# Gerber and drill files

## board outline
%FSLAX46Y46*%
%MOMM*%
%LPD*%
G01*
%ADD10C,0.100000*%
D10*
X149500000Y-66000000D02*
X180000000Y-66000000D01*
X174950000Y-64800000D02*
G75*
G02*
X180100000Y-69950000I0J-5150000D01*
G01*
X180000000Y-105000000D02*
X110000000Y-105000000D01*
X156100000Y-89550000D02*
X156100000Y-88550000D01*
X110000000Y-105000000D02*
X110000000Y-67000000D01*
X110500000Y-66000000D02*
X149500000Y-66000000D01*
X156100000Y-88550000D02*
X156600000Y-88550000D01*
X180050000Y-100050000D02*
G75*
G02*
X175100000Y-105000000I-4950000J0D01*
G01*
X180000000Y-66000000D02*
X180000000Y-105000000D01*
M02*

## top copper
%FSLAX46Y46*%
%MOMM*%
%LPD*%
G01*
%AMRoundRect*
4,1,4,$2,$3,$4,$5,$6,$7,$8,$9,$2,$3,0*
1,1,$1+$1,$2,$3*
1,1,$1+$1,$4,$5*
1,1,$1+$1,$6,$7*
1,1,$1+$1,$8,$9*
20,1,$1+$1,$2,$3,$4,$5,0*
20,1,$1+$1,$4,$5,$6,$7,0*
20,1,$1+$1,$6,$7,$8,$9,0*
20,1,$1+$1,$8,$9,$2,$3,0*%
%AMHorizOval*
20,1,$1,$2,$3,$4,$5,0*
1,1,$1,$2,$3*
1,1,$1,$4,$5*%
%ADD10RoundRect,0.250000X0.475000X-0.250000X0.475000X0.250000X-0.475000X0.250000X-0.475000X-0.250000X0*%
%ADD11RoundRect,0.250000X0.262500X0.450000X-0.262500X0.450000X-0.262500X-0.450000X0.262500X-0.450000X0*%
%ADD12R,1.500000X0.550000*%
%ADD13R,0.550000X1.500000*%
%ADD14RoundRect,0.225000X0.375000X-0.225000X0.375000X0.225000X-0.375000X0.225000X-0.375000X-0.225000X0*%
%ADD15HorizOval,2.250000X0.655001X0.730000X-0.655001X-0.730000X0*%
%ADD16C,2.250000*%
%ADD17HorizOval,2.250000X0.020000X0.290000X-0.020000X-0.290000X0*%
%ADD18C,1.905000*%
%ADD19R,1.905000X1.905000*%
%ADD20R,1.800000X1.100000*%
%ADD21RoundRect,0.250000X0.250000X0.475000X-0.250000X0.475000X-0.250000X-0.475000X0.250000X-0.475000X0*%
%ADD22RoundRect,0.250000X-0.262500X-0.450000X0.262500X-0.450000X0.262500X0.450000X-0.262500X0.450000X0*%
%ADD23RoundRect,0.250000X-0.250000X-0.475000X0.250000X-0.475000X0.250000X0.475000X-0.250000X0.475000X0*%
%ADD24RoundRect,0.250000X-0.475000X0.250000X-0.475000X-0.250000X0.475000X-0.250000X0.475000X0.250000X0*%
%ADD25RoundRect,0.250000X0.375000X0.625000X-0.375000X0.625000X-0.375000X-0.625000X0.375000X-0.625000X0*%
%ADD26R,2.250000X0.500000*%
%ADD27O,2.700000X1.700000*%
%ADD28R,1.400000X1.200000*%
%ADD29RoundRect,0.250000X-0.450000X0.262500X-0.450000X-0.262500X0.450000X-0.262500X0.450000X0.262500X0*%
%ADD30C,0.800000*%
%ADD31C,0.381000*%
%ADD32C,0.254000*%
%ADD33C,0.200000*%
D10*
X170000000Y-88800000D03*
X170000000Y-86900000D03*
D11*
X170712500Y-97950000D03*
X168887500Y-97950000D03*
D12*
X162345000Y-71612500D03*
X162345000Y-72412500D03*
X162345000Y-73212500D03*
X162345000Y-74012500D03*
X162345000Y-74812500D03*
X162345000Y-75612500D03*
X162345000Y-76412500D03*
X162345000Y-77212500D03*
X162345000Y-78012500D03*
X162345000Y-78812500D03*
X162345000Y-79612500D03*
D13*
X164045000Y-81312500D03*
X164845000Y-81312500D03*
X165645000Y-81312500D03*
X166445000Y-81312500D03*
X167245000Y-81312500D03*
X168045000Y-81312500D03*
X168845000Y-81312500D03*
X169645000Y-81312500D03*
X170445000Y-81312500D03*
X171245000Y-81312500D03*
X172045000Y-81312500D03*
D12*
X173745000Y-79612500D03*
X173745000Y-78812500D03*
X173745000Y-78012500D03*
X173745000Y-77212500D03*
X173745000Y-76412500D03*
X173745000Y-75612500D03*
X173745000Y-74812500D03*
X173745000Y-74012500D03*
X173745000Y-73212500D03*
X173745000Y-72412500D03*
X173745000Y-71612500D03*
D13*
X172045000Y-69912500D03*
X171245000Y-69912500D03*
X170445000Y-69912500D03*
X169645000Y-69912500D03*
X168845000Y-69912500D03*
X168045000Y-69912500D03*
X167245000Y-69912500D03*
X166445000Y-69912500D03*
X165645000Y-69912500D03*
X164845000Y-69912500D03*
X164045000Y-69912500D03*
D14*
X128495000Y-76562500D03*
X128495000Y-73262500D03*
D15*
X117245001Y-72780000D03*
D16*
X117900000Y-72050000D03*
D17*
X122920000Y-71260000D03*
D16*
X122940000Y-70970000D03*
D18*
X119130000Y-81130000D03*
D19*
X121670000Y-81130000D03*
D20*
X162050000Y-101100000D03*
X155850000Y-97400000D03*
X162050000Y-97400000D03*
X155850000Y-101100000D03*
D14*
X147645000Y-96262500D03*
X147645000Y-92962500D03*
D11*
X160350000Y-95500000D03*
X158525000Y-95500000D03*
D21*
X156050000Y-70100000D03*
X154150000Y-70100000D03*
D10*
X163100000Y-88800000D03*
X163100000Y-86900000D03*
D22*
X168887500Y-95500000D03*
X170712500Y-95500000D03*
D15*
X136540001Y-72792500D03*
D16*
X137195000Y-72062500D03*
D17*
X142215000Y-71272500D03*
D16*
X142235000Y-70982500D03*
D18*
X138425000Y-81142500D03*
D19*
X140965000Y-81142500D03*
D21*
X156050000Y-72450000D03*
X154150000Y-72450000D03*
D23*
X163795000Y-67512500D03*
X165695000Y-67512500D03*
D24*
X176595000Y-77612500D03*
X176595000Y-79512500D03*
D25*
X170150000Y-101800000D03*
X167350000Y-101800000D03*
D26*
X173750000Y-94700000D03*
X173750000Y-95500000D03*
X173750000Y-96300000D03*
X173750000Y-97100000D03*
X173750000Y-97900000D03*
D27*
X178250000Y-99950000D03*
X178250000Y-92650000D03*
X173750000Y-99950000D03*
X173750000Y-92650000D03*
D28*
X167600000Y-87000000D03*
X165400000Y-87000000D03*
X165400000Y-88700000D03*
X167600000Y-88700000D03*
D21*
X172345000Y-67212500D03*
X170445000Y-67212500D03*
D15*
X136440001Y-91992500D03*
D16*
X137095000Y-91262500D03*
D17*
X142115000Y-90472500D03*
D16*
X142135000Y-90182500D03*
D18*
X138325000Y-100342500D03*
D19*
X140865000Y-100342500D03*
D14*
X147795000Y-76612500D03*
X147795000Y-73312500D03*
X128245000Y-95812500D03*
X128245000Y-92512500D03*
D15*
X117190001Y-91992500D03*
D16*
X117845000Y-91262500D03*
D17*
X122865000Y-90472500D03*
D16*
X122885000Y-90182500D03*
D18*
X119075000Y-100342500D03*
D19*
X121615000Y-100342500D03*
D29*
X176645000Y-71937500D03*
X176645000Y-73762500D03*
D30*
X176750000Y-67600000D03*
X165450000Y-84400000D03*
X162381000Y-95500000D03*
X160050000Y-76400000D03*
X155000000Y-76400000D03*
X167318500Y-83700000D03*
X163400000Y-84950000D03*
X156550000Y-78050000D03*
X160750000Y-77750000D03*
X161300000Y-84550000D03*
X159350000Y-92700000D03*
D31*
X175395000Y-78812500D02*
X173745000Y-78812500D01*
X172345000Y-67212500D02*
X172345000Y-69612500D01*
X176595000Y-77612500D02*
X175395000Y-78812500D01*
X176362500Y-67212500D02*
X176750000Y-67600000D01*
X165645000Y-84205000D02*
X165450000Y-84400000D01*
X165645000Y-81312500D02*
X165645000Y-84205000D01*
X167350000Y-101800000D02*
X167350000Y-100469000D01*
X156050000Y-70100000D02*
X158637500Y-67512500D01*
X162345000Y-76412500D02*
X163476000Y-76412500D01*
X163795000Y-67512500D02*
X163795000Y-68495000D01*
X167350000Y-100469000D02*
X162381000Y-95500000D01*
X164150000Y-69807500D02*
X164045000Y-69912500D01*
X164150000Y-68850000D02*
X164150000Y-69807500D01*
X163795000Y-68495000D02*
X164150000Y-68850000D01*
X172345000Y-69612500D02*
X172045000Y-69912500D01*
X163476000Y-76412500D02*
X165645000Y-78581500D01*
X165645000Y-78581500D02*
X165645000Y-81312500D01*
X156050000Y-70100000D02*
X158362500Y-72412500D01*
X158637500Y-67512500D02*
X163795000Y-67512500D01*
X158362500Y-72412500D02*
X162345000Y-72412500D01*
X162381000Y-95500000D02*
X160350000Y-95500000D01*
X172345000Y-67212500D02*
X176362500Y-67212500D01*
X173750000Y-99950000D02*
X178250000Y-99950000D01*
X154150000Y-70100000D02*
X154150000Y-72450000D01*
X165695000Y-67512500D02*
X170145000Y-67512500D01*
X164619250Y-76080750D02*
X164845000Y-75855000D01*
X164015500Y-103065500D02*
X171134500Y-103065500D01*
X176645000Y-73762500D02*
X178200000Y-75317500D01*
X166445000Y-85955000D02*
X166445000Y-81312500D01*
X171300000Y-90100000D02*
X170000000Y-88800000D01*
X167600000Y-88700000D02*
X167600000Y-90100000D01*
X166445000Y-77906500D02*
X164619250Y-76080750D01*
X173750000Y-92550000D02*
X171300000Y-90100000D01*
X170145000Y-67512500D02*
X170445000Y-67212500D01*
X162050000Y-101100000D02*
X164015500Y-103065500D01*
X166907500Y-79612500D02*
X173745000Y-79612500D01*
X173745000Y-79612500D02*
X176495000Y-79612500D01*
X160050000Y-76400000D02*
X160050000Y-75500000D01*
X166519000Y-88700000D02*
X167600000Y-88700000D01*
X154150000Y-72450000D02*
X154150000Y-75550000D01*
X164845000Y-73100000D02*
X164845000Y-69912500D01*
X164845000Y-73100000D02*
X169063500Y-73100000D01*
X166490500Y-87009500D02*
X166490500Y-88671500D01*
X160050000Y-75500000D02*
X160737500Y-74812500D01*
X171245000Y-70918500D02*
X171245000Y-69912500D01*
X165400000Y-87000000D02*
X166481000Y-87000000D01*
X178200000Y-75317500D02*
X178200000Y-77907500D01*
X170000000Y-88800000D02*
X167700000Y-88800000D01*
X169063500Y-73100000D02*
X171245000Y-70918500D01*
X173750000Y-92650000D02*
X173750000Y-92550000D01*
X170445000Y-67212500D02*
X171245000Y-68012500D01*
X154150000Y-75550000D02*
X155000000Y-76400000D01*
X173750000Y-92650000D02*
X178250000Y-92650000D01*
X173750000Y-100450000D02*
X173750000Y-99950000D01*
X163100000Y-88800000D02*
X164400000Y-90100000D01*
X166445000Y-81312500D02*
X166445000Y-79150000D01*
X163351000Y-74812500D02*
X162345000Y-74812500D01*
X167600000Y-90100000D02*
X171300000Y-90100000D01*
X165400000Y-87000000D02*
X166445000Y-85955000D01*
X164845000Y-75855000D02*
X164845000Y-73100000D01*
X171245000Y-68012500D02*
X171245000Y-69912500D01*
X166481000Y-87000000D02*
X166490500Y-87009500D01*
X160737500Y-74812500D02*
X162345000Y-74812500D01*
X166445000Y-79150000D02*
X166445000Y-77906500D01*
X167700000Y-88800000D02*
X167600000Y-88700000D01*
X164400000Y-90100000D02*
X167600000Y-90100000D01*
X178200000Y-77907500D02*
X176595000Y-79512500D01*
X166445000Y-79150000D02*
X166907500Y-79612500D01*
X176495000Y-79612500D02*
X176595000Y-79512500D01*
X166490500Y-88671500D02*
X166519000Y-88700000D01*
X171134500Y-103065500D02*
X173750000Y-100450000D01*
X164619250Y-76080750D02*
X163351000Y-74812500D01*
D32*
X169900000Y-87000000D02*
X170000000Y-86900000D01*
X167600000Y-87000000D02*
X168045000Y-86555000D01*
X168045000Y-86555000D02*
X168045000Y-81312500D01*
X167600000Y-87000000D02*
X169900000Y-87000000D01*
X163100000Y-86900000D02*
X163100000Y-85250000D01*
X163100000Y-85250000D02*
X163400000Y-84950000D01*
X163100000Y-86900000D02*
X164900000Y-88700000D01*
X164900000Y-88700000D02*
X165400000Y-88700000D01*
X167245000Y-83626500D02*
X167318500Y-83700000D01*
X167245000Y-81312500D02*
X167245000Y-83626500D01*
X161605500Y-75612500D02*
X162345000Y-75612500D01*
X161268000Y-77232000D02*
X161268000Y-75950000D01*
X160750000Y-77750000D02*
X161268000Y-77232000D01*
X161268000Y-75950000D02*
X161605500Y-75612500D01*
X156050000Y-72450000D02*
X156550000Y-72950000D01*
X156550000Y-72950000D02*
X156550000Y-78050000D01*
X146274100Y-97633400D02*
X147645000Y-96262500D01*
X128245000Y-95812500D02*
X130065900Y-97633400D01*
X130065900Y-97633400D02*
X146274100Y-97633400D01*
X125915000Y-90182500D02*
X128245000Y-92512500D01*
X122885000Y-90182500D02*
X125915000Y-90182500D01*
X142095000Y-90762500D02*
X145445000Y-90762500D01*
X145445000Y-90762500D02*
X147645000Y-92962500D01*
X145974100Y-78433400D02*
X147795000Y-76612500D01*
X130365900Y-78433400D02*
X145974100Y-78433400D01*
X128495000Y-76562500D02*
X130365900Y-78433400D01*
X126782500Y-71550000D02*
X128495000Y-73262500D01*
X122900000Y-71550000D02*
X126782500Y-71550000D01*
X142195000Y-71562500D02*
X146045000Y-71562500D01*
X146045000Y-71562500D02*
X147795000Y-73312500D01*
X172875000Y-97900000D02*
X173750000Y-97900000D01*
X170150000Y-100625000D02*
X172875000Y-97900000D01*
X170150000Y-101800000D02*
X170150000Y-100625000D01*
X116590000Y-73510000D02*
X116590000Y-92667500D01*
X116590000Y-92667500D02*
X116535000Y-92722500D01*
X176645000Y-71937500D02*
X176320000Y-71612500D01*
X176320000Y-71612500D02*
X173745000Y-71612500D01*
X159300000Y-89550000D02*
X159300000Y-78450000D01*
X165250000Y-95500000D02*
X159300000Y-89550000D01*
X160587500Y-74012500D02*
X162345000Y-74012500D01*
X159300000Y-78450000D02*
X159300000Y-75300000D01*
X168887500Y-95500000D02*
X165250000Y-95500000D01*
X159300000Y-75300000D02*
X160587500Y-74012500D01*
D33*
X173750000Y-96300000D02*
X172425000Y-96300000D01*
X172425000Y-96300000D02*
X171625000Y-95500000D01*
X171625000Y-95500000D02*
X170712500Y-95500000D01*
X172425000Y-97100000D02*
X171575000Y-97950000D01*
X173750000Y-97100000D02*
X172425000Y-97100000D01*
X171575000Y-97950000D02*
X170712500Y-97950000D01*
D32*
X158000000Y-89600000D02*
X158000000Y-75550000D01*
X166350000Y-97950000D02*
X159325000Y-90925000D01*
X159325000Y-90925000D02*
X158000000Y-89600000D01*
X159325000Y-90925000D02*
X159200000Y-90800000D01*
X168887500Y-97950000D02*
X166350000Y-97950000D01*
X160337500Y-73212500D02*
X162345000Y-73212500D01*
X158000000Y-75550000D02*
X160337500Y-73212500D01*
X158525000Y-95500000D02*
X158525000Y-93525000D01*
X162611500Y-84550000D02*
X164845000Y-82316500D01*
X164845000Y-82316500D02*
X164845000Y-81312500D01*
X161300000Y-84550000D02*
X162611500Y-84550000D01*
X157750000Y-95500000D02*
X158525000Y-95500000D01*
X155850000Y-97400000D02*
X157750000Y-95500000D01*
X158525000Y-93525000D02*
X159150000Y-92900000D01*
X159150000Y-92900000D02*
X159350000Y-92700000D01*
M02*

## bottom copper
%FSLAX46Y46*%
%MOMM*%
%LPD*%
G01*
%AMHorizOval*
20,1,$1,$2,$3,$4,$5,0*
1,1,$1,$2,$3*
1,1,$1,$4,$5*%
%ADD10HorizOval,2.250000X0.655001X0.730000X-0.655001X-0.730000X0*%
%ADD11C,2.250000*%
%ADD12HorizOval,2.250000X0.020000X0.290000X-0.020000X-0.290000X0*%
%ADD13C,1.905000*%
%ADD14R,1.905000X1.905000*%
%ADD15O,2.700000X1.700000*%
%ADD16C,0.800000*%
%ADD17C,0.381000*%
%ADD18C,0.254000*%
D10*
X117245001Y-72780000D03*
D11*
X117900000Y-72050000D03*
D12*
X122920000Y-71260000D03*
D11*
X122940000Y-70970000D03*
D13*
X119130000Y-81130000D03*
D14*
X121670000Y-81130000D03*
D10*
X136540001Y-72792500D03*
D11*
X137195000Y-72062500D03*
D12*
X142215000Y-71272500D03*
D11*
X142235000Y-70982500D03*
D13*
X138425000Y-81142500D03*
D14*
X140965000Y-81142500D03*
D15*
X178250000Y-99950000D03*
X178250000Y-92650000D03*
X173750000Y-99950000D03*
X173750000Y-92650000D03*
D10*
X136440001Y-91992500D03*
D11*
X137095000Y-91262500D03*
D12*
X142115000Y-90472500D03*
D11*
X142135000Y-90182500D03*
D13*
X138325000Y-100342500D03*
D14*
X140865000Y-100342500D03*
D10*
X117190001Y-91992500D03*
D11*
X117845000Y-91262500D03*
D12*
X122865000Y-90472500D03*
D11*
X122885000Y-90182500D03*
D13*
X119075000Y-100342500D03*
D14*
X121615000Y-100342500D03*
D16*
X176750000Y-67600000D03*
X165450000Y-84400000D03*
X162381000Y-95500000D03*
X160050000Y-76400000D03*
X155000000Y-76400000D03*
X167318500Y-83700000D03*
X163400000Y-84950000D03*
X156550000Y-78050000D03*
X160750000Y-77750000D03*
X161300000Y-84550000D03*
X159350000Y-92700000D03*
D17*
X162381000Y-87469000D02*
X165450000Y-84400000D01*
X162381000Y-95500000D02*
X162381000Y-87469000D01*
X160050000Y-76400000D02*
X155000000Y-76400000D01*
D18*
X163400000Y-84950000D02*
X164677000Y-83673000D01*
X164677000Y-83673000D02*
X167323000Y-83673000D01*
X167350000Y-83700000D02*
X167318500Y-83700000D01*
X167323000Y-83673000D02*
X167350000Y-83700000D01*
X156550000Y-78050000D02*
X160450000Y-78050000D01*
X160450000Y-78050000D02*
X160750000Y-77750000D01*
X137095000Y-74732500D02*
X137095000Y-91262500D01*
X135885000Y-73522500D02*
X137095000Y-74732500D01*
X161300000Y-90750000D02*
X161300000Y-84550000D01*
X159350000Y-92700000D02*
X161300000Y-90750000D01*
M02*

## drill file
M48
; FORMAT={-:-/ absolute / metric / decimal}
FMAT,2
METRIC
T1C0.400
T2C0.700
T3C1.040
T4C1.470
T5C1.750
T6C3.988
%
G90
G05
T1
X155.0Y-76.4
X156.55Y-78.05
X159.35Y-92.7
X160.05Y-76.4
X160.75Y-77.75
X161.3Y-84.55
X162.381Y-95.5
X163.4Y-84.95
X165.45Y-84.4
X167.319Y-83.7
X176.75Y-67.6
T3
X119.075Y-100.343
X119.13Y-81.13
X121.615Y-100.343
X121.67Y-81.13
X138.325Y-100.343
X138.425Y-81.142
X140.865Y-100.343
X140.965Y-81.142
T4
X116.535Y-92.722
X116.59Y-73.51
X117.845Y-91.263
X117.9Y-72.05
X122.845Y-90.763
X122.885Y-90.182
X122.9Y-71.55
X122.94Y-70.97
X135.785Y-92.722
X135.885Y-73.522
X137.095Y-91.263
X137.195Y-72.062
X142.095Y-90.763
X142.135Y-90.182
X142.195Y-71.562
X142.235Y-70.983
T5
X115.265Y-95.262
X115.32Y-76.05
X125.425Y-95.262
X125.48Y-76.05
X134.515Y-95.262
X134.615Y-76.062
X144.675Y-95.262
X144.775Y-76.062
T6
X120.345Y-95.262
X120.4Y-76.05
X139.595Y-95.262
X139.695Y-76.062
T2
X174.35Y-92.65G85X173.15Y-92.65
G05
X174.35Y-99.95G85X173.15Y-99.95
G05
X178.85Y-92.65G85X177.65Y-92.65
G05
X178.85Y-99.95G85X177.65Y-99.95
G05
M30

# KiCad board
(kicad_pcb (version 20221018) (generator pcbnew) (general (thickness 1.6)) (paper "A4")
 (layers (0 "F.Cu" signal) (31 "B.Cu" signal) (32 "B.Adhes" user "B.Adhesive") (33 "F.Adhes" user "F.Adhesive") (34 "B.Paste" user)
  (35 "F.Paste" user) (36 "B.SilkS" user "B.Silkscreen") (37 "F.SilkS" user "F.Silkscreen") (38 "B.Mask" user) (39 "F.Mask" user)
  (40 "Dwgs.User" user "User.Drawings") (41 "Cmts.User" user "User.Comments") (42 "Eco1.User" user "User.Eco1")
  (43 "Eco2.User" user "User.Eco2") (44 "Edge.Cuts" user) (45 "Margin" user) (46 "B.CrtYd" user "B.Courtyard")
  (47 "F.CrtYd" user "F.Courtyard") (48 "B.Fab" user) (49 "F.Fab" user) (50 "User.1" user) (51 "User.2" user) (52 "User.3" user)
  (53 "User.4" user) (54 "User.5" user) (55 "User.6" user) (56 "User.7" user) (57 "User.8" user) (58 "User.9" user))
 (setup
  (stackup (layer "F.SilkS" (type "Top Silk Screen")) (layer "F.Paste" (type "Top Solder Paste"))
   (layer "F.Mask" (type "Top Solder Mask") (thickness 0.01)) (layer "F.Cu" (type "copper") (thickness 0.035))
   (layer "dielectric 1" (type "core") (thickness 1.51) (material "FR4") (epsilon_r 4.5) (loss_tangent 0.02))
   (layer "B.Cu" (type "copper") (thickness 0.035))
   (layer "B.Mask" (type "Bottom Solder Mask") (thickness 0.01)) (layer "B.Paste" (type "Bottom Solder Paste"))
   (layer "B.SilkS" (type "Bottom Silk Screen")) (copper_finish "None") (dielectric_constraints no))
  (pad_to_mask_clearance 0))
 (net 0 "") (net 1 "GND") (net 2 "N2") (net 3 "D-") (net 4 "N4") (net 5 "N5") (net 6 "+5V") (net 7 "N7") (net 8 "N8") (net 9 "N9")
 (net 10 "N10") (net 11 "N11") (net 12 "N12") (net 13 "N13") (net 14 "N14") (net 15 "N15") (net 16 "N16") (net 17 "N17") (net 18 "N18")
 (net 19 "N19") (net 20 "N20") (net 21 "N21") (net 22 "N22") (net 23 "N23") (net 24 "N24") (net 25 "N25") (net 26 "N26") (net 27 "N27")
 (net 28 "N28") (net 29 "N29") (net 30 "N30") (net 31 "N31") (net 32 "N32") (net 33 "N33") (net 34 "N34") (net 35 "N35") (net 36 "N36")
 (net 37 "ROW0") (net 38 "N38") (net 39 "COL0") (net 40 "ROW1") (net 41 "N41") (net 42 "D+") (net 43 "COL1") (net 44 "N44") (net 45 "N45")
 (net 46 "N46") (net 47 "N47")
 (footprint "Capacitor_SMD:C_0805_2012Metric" (layer "F.Cu") (at 170 87.85 90)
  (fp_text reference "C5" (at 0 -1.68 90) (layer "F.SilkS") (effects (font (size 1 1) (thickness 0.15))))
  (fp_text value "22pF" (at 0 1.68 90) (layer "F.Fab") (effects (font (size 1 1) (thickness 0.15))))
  (pad "1" smd roundrect (at -0.95 0 90) (size 1 1.45) (layers "F.Cu" "F.Paste" "F.Mask") (roundrect_rratio 0.25) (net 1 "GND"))
  (pad "2" smd roundrect (at 0.95 0 90) (size 1 1.45) (layers "F.Cu" "F.Paste" "F.Mask") (roundrect_rratio 0.25) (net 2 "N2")))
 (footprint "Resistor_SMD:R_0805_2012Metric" (layer "F.Cu") (at 169.8 97.95 180)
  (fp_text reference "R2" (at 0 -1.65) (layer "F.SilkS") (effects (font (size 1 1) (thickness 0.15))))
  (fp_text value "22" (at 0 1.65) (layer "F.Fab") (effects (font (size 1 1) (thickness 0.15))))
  (pad "1" smd roundrect (at -0.9125 0 180) (size 1.025 1.4) (layers "F.Cu" "F.Paste" "F.Mask") (roundrect_rratio 0.243902) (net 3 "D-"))
  (pad "2" smd roundrect (at 0.9125 0 180) (size 1.025 1.4) (layers "F.Cu" "F.Paste" "F.Mask") (roundrect_rratio 0.243902) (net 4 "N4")))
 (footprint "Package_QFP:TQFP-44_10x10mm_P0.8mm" (layer "F.Cu") (at 168.045 75.6125)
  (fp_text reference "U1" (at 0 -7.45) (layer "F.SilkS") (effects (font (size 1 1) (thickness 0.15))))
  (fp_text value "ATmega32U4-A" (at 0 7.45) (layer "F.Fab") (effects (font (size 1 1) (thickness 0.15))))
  (pad "1" smd rect (at -5.7 -4) (size 1.5 0.55) (layers "F.Cu" "F.Paste" "F.Mask") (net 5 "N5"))
  (pad "2" smd rect (at -5.7 -3.2) (size 1.5 0.55) (layers "F.Cu" "F.Paste" "F.Mask") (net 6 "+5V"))
  (pad "3" smd rect (at -5.7 -2.4) (size 1.5 0.55) (layers "F.Cu" "F.Paste" "F.Mask") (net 4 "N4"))
  (pad "4" smd rect (at -5.7 -1.6) (size 1.5 0.55) (layers "F.Cu" "F.Paste" "F.Mask") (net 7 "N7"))
  (pad "5" smd rect (at -5.7 -0.8) (size 1.5 0.55) (layers "F.Cu" "F.Paste" "F.Mask") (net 1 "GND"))
  (pad "6" smd rect (at -5.7 0) (size 1.5 0.55) (layers "F.Cu" "F.Paste" "F.Mask") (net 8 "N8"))
  (pad "7" smd rect (at -5.7 0.8) (size 1.5 0.55) (layers "F.Cu" "F.Paste" "F.Mask") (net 6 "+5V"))
  (pad "8" smd rect (at -5.7 1.6) (size 1.5 0.55) (layers "F.Cu" "F.Paste" "F.Mask") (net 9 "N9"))
  (pad "9" smd rect (at -5.7 2.4) (size 1.5 0.55) (layers "F.Cu" "F.Paste" "F.Mask") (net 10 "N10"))
  (pad "10" smd rect (at -5.7 3.2) (size 1.5 0.55) (layers "F.Cu" "F.Paste" "F.Mask") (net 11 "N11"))
  (pad "11" smd rect (at -5.7 4) (size 1.5 0.55) (layers "F.Cu" "F.Paste" "F.Mask") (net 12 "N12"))
  (pad "12" smd rect (at -4 5.7 90) (size 1.5 0.55) (layers "F.Cu" "F.Paste" "F.Mask") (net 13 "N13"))
  (pad "13" smd rect (at -3.2 5.7 90) (size 1.5 0.55) (layers "F.Cu" "F.Paste" "F.Mask") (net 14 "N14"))
  (pad "14" smd rect (at -2.4 5.7 90) (size 1.5 0.55) (layers "F.Cu" "F.Paste" "F.Mask") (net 6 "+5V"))
  (pad "15" smd rect (at -1.6 5.7 90) (size 1.5 0.55) (layers "F.Cu" "F.Paste" "F.Mask") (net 1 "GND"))
  (pad "16" smd rect (at -0.8 5.7 90) (size 1.5 0.55) (layers "F.Cu" "F.Paste" "F.Mask") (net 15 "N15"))
  (pad "17" smd rect (at 0 5.7 90) (size 1.5 0.55) (layers "F.Cu" "F.Paste" "F.Mask") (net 2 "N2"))
  (pad "18" smd rect (at 0.8 5.7 90) (size 1.5 0.55) (layers "F.Cu" "F.Paste" "F.Mask") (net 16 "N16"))
  (pad "19" smd rect (at 1.6 5.7 90) (size 1.5 0.55) (layers "F.Cu" "F.Paste" "F.Mask") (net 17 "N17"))
  (pad "20" smd rect (at 2.4 5.7 90) (size 1.5 0.55) (layers "F.Cu" "F.Paste" "F.Mask") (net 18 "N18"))
  (pad "21" smd rect (at 3.2 5.7 90) (size 1.5 0.55) (layers "F.Cu" "F.Paste" "F.Mask") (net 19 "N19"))
  (pad "22" smd rect (at 4 5.7 90) (size 1.5 0.55) (layers "F.Cu" "F.Paste" "F.Mask") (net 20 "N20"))
  (pad "23" smd rect (at 5.7 4) (size 1.5 0.55) (layers "F.Cu" "F.Paste" "F.Mask") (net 1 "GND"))
  (pad "24" smd rect (at 5.7 3.2) (size 1.5 0.55) (layers "F.Cu" "F.Paste" "F.Mask") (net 6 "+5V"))
  (pad "25" smd rect (at 5.7 2.4) (size 1.5 0.55) (layers "F.Cu" "F.Paste" "F.Mask") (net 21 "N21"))
  (pad "26" smd rect (at 5.7 1.6) (size 1.5 0.55) (layers "F.Cu" "F.Paste" "F.Mask") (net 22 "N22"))
  (pad "27" smd rect (at 5.7 0.8) (size 1.5 0.55) (layers "F.Cu" "F.Paste" "F.Mask") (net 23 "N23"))
  (pad "28" smd rect (at 5.7 0) (size 1.5 0.55) (layers "F.Cu" "F.Paste" "F.Mask") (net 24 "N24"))
  (pad "29" smd rect (at 5.7 -0.8) (size 1.5 0.55) (layers "F.Cu" "F.Paste" "F.Mask") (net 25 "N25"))
  (pad "30" smd rect (at 5.7 -1.6) (size 1.5 0.55) (layers "F.Cu" "F.Paste" "F.Mask") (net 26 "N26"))
  (pad "31" smd rect (at 5.7 -2.4) (size 1.5 0.55) (layers "F.Cu" "F.Paste" "F.Mask") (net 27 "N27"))
  (pad "32" smd rect (at 5.7 -3.2) (size 1.5 0.55) (layers "F.Cu" "F.Paste" "F.Mask") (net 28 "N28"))
  (pad "33" smd rect (at 5.7 -4) (size 1.5 0.55) (layers "F.Cu" "F.Paste" "F.Mask") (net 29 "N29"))
  (pad "34" smd rect (at 4 -5.7 90) (size 1.5 0.55) (layers "F.Cu" "F.Paste" "F.Mask") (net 6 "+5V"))
  (pad "35" smd rect (at 3.2 -5.7 90) (size 1.5 0.55) (layers "F.Cu" "F.Paste" "F.Mask") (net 1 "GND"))
  (pad "36" smd rect (at 2.4 -5.7 90) (size 1.5 0.55) (layers "F.Cu" "F.Paste" "F.Mask") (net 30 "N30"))
  (pad "37" smd rect (at 1.6 -5.7 90) (size 1.5 0.55) (layers "F.Cu" "F.Paste" "F.Mask") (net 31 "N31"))
  (pad "38" smd rect (at 0.8 -5.7 90) (size 1.5 0.55) (layers "F.Cu" "F.Paste" "F.Mask") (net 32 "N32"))
  (pad "39" smd rect (at 0 -5.7 90) (size 1.5 0.55) (layers "F.Cu" "F.Paste" "F.Mask") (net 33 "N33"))
  (pad "40" smd rect (at -0.8 -5.7 90) (size 1.5 0.55) (layers "F.Cu" "F.Paste" "F.Mask") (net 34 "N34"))
  (pad "41" smd rect (at -1.6 -5.7 90) (size 1.5 0.55) (layers "F.Cu" "F.Paste" "F.Mask") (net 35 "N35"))
  (pad "42" smd rect (at -2.4 -5.7 90) (size 1.5 0.55) (layers "F.Cu" "F.Paste" "F.Mask") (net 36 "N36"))
  (pad "43" smd rect (at -3.2 -5.7 90) (size 1.5 0.55) (layers "F.Cu" "F.Paste" "F.Mask") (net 1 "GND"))
  (pad "44" smd rect (at -4 -5.7 90) (size 1.5 0.55) (layers "F.Cu" "F.Paste" "F.Mask") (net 6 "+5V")))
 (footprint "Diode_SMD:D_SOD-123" (layer "F.Cu") (at 128.495 74.9125 90)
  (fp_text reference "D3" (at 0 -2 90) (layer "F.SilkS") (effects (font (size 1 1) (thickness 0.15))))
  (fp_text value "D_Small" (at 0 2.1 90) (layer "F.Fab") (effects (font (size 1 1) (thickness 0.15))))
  (pad "1" smd roundrect (at -1.65 0 90) (size 0.9 1.2) (layers "F.Cu" "F.Paste" "F.Mask") (roundrect_rratio 0.25) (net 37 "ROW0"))
  (pad "2" smd roundrect (at 1.65 0 90) (size 0.9 1.2) (layers "F.Cu" "F.Paste" "F.Mask") (roundrect_rratio 0.25) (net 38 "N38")))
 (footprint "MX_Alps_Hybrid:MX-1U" (layer "F.Cu") (at 120.4 76.05)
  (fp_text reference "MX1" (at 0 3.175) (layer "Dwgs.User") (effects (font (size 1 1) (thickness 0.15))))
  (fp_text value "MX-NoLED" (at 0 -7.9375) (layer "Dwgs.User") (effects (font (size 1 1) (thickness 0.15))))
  (pad "" np_thru_hole circle (at -5.08 0 48.0996) (size 1.75 1.75) (drill 1.75) (layers "*.Cu" "*.Mask"))
  (pad "" np_thru_hole circle (at 0 0) (size 3.9878 3.9878) (drill 3.9878) (layers "*.Cu" "*.Mask"))
  (pad "" np_thru_hole circle (at 5.08 0 48.0996) (size 1.75 1.75) (drill 1.75) (layers "*.Cu" "*.Mask"))
  (pad "1" thru_hole oval (at -3.81 -2.54 48.0996) (size 4.211556 2.25) (drill 1.47 (offset 0.980778 0)) (layers "*.Cu" "B.Mask")
   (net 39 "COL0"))
  (pad "1" thru_hole circle (at -2.5 -4) (size 2.25 2.25) (drill 1.47) (layers "*.Cu" "B.Mask") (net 39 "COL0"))
  (pad "2" thru_hole oval (at 2.5 -4.5 86.0548) (size 2.831378 2.25) (drill 1.47 (offset 0.290689 0)) (layers "*.Cu" "B.Mask")
   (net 38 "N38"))
  (pad "2" thru_hole circle (at 2.54 -5.08) (size 2.25 2.25) (drill 1.47) (layers "*.Cu" "B.Mask") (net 38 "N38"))
  (pad "3" thru_hole circle (at -1.27 5.08) (size 1.905 1.905) (drill 1.04) (layers "*.Cu" "B.Mask"))
  (pad "4" thru_hole rect (at 1.27 5.08) (size 1.905 1.905) (drill 1.04) (layers "*.Cu" "B.Mask")))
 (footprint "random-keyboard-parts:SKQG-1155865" (layer "F.Cu") (at 158.95 99.25)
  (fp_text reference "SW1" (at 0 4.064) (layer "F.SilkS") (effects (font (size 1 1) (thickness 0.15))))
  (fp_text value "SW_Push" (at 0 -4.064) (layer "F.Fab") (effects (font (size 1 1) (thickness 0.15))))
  (pad "1" smd rect (at 3.1 1.85) (size 1.8 1.1) (layers "F.Cu" "F.Paste" "F.Mask") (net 1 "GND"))
  (pad "2" smd rect (at -3.1 -1.85) (size 1.8 1.1) (layers "F.Cu" "F.Paste" "F.Mask") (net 14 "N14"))
  (pad "3" smd rect (at 3.1 -1.85) (size 1.8 1.1) (layers "F.Cu" "F.Paste" "F.Mask"))
  (pad "4" smd rect (at -3.1 1.85) (size 1.8 1.1) (layers "F.Cu" "F.Paste" "F.Mask")))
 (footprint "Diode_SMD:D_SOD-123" (layer "F.Cu") (at 147.645 94.6125 90)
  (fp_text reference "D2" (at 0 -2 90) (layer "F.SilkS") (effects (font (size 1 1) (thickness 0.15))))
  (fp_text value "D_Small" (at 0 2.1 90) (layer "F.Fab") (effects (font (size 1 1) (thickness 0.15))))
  (pad "1" smd roundrect (at -1.65 0 90) (size 0.9 1.2) (layers "F.Cu" "F.Paste" "F.Mask") (roundrect_rratio 0.25) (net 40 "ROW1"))
  (pad "2" smd roundrect (at 1.65 0 90) (size 0.9 1.2) (layers "F.Cu" "F.Paste" "F.Mask") (roundrect_rratio 0.25) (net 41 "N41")))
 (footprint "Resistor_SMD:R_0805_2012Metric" (layer "F.Cu") (at 159.4375 95.5 180)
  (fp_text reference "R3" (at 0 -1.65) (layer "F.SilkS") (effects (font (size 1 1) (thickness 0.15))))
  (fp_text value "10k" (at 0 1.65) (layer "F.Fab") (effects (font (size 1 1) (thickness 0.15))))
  (pad "1" smd roundrect (at -0.9125 0 180) (size 1.025 1.4) (layers "F.Cu" "F.Paste" "F.Mask") (roundrect_rratio 0.243902) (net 6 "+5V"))
  (pad "2" smd roundrect (at 0.9125 0 180) (size 1.025 1.4) (layers "F.Cu" "F.Paste" "F.Mask") (roundrect_rratio 0.243902) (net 14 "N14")))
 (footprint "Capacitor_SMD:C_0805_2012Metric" (layer "F.Cu") (at 155.1 70.1 180)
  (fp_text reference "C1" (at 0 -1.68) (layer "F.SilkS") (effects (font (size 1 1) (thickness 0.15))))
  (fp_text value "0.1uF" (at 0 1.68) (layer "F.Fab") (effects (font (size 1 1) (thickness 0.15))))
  (pad "1" smd roundrect (at -0.95 0 180) (size 1 1.45) (layers "F.Cu" "F.Paste" "F.Mask") (roundrect_rratio 0.25) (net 6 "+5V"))
  (pad "2" smd roundrect (at 0.95 0 180) (size 1 1.45) (layers "F.Cu" "F.Paste" "F.Mask") (roundrect_rratio 0.25) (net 1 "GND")))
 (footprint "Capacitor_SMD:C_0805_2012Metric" (layer "F.Cu") (at 163.1 87.85 90)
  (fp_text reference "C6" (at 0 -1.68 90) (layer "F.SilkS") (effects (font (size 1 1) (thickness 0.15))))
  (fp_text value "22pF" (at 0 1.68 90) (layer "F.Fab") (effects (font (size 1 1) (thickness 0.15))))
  (pad "1" smd roundrect (at -0.95 0 90) (size 1 1.45) (layers "F.Cu" "F.Paste" "F.Mask") (roundrect_rratio 0.25) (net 1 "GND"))
  (pad "2" smd roundrect (at 0.95 0 90) (size 1 1.45) (layers "F.Cu" "F.Paste" "F.Mask") (roundrect_rratio 0.25) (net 15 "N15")))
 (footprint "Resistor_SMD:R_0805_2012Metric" (layer "F.Cu") (at 169.8 95.5)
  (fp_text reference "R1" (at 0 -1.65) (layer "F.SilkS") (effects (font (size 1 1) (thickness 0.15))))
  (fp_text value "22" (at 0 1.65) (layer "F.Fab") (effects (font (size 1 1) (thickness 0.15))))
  (pad "1" smd roundrect (at -0.9125 0) (size 1.025 1.4) (layers "F.Cu" "F.Paste" "F.Mask") (roundrect_rratio 0.243902) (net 7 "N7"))
  (pad "2" smd roundrect (at 0.9125 0) (size 1.025 1.4) (layers "F.Cu" "F.Paste" "F.Mask") (roundrect_rratio 0.243902) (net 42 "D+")))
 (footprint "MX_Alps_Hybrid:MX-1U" (layer "F.Cu") (at 139.695 76.0625)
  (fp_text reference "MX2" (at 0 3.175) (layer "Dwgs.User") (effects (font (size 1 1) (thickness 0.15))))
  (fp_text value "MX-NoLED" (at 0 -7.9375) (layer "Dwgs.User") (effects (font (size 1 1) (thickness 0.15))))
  (pad "" np_thru_hole circle (at -5.08 0 48.0996) (size 1.75 1.75) (drill 1.75) (layers "*.Cu" "*.Mask"))
  (pad "" np_thru_hole circle (at 0 0) (size 3.9878 3.9878) (drill 3.9878) (layers "*.Cu" "*.Mask"))
  (pad "" np_thru_hole circle (at 5.08 0 48.0996) (size 1.75 1.75) (drill 1.75) (layers "*.Cu" "*.Mask"))
  (pad "1" thru_hole oval (at -3.81 -2.54 48.0996) (size 4.211556 2.25) (drill 1.47 (offset 0.980778 0)) (layers "*.Cu" "B.Mask")
   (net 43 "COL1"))
  (pad "1" thru_hole circle (at -2.5 -4) (size 2.25 2.25) (drill 1.47) (layers "*.Cu" "B.Mask") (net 43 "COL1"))
  (pad "2" thru_hole oval (at 2.5 -4.5 86.0548) (size 2.831378 2.25) (drill 1.47 (offset 0.290689 0)) (layers "*.Cu" "B.Mask")
   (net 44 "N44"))
  (pad "2" thru_hole circle (at 2.54 -5.08) (size 2.25 2.25) (drill 1.47) (layers "*.Cu" "B.Mask") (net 44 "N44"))
  (pad "3" thru_hole circle (at -1.27 5.08) (size 1.905 1.905) (drill 1.04) (layers "*.Cu" "B.Mask"))
  (pad "4" thru_hole rect (at 1.27 5.08) (size 1.905 1.905) (drill 1.04) (layers "*.Cu" "B.Mask")))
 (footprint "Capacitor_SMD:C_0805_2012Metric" (layer "F.Cu") (at 155.1 72.45 180)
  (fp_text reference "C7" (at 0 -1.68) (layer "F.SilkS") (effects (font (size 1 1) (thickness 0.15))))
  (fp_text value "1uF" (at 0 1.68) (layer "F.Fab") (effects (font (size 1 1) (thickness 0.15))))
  (pad "1" smd roundrect (at -0.95 0 180) (size 1 1.45) (layers "F.Cu" "F.Paste" "F.Mask") (roundrect_rratio 0.25) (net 8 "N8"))
  (pad "2" smd roundrect (at 0.95 0 180) (size 1 1.45) (layers "F.Cu" "F.Paste" "F.Mask") (roundrect_rratio 0.25) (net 1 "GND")))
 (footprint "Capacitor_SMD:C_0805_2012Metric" (layer "F.Cu") (at 164.745 67.5125)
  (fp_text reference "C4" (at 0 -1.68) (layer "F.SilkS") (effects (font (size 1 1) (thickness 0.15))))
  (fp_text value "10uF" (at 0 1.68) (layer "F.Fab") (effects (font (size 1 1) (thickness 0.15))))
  (pad "1" smd roundrect (at -0.95 0) (size 1 1.45) (layers "F.Cu" "F.Paste" "F.Mask") (roundrect_rratio 0.25) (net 6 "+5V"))
  (pad "2" smd roundrect (at 0.95 0) (size 1 1.45) (layers "F.Cu" "F.Paste" "F.Mask") (roundrect_rratio 0.25) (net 1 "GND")))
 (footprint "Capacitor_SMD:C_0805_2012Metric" (layer "F.Cu") (at 176.595 78.5625 -90)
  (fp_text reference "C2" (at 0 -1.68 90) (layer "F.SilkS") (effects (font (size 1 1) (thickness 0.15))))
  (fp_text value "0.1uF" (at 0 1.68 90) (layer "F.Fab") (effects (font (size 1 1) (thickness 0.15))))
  (pad "1" smd roundrect (at -0.95 0 270) (size 1 1.45) (layers "F.Cu" "F.Paste" "F.Mask") (roundrect_rratio 0.25) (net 6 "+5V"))
  (pad "2" smd roundrect (at 0.95 0 270) (size 1 1.45) (layers "F.Cu" "F.Paste" "F.Mask") (roundrect_rratio 0.25) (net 1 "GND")))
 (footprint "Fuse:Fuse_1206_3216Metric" (layer "F.Cu") (at 168.75 101.8 180)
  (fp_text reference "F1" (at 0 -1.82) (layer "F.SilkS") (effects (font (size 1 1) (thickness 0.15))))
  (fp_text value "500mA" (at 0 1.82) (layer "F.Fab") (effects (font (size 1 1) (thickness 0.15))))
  (pad "1" smd roundrect (at -1.4 0 180) (size 1.25 1.75) (layers "F.Cu" "F.Paste" "F.Mask") (roundrect_rratio 0.2) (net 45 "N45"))
  (pad "2" smd roundrect (at 1.4 0 180) (size 1.25 1.75) (layers "F.Cu" "F.Paste" "F.Mask") (roundrect_rratio 0.2) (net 6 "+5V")))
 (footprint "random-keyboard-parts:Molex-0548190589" (layer "F.Cu") (at 178.25 96.3 180)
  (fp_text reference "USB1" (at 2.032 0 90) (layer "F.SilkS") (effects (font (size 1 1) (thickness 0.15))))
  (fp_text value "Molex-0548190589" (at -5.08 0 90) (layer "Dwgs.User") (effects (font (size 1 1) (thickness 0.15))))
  (pad "1" smd rect (at 4.5 1.6 180) (size 2.25 0.5) (layers "F.Cu" "F.Paste" "F.Mask") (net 1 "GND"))
  (pad "2" smd rect (at 4.5 0.8 180) (size 2.25 0.5) (layers "F.Cu" "F.Paste" "F.Mask") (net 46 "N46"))
  (pad "3" smd rect (at 4.5 0 180) (size 2.25 0.5) (layers "F.Cu" "F.Paste" "F.Mask") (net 42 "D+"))
  (pad "4" smd rect (at 4.5 -0.8 180) (size 2.25 0.5) (layers "F.Cu" "F.Paste" "F.Mask") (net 3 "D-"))
  (pad "5" smd rect (at 4.5 -1.6 180) (size 2.25 0.5) (layers "F.Cu" "F.Paste" "F.Mask") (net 45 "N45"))
  (pad "6" thru_hole oval (at 0 -3.65 180) (size 2.7 1.7) (drill oval 1.9 0.7) (layers "*.Cu" "*.Mask") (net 1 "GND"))
  (pad "6" thru_hole oval (at 0 3.65 180) (size 2.7 1.7) (drill oval 1.9 0.7) (layers "*.Cu" "*.Mask") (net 1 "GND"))
  (pad "6" thru_hole oval (at 4.5 -3.65 180) (size 2.7 1.7) (drill oval 1.9 0.7) (layers "*.Cu" "*.Mask") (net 1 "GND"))
  (pad "6" thru_hole oval (at 4.5 3.65 180) (size 2.7 1.7) (drill oval 1.9 0.7) (layers "*.Cu" "*.Mask") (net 1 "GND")))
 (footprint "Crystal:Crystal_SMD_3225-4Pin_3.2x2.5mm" (layer "F.Cu") (at 166.5 87.85 180)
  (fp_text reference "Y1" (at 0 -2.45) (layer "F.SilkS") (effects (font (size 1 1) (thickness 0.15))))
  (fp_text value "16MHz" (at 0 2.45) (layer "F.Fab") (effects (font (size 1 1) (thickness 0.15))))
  (pad "1" smd rect (at -1.1 0.85 180) (size 1.4 1.2) (layers "F.Cu" "F.Paste" "F.Mask") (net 2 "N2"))
  (pad "2" smd rect (at 1.1 0.85 180) (size 1.4 1.2) (layers "F.Cu" "F.Paste" "F.Mask") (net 1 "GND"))
  (pad "3" smd rect (at 1.1 -0.85 180) (size 1.4 1.2) (layers "F.Cu" "F.Paste" "F.Mask") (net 15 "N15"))
  (pad "4" smd rect (at -1.1 -0.85 180) (size 1.4 1.2) (layers "F.Cu" "F.Paste" "F.Mask") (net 1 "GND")))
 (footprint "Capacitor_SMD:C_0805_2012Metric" (layer "F.Cu") (at 171.395 67.2125 180)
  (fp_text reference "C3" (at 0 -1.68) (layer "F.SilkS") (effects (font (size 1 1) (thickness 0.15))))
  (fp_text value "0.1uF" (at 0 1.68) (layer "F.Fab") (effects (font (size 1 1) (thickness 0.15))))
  (pad "1" smd roundrect (at -0.95 0 180) (size 1 1.45) (layers "F.Cu" "F.Paste" "F.Mask") (roundrect_rratio 0.25) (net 6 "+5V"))
  (pad "2" smd roundrect (at 0.95 0 180) (size 1 1.45) (layers "F.Cu" "F.Paste" "F.Mask") (roundrect_rratio 0.25) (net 1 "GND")))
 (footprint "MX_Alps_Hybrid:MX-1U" (layer "F.Cu") (at 139.595 95.2625)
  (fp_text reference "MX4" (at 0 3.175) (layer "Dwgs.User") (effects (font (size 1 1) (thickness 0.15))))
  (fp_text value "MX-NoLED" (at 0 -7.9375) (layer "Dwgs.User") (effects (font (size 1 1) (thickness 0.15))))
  (pad "" np_thru_hole circle (at -5.08 0 48.0996) (size 1.75 1.75) (drill 1.75) (layers "*.Cu" "*.Mask"))
  (pad "" np_thru_hole circle (at 0 0) (size 3.9878 3.9878) (drill 3.9878) (layers "*.Cu" "*.Mask"))
  (pad "" np_thru_hole circle (at 5.08 0 48.0996) (size 1.75 1.75) (drill 1.75) (layers "*.Cu" "*.Mask"))
  (pad "1" thru_hole oval (at -3.81 -2.54 48.0996) (size 4.211556 2.25) (drill 1.47 (offset 0.980778 0)) (layers "*.Cu" "B.Mask")
   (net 43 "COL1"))
  (pad "1" thru_hole circle (at -2.5 -4) (size 2.25 2.25) (drill 1.47) (layers "*.Cu" "B.Mask") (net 43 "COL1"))
  (pad "2" thru_hole oval (at 2.5 -4.5 86.0548) (size 2.831378 2.25) (drill 1.47 (offset 0.290689 0)) (layers "*.Cu" "B.Mask")
   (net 41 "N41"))
  (pad "2" thru_hole circle (at 2.54 -5.08) (size 2.25 2.25) (drill 1.47) (layers "*.Cu" "B.Mask") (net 41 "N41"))
  (pad "3" thru_hole circle (at -1.27 5.08) (size 1.905 1.905) (drill 1.04) (layers "*.Cu" "B.Mask"))
  (pad "4" thru_hole rect (at 1.27 5.08) (size 1.905 1.905) (drill 1.04) (layers "*.Cu" "B.Mask")))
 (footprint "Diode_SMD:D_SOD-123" (layer "F.Cu") (at 147.795 74.9625 90)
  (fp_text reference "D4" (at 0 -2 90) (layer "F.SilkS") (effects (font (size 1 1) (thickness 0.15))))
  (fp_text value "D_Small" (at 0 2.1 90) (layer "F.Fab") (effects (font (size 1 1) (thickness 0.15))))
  (pad "1" smd roundrect (at -1.65 0 90) (size 0.9 1.2) (layers "F.Cu" "F.Paste" "F.Mask") (roundrect_rratio 0.25) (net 37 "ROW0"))
  (pad "2" smd roundrect (at 1.65 0 90) (size 0.9 1.2) (layers "F.Cu" "F.Paste" "F.Mask") (roundrect_rratio 0.25) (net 44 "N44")))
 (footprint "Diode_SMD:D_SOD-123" (layer "F.Cu") (at 128.245 94.1625 90)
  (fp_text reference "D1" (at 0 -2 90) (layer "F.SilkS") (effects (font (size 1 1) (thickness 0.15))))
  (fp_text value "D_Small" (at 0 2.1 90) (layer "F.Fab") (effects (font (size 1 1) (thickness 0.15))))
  (pad "1" smd roundrect (at -1.65 0 90) (size 0.9 1.2) (layers "F.Cu" "F.Paste" "F.Mask") (roundrect_rratio 0.25) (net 40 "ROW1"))
  (pad "2" smd roundrect (at 1.65 0 90) (size 0.9 1.2) (layers "F.Cu" "F.Paste" "F.Mask") (roundrect_rratio 0.25) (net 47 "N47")))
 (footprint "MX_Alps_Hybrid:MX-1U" (layer "F.Cu") (at 120.345 95.2625)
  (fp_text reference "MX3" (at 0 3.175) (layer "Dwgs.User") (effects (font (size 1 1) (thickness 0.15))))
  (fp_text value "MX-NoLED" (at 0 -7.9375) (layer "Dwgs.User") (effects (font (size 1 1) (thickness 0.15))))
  (pad "" np_thru_hole circle (at -5.08 0 48.0996) (size 1.75 1.75) (drill 1.75) (layers "*.Cu" "*.Mask"))
  (pad "" np_thru_hole circle (at 0 0) (size 3.9878 3.9878) (drill 3.9878) (layers "*.Cu" "*.Mask"))
  (pad "" np_thru_hole circle (at 5.08 0 48.0996) (size 1.75 1.75) (drill 1.75) (layers "*.Cu" "*.Mask"))
  (pad "1" thru_hole oval (at -3.81 -2.54 48.0996) (size 4.211556 2.25) (drill 1.47 (offset 0.980778 0)) (layers "*.Cu" "B.Mask")
   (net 39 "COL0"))
  (pad "1" thru_hole circle (at -2.5 -4) (size 2.25 2.25) (drill 1.47) (layers "*.Cu" "B.Mask") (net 39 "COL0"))
  (pad "2" thru_hole oval (at 2.5 -4.5 86.0548) (size 2.831378 2.25) (drill 1.47 (offset 0.290689 0)) (layers "*.Cu" "B.Mask")
   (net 47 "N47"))
  (pad "2" thru_hole circle (at 2.54 -5.08) (size 2.25 2.25) (drill 1.47) (layers "*.Cu" "B.Mask") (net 47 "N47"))
  (pad "3" thru_hole circle (at -1.27 5.08) (size 1.905 1.905) (drill 1.04) (layers "*.Cu" "B.Mask"))
  (pad "4" thru_hole rect (at 1.27 5.08) (size 1.905 1.905) (drill 1.04) (layers "*.Cu" "B.Mask")))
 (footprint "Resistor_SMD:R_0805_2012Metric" (layer "F.Cu") (at 176.645 72.85 -90)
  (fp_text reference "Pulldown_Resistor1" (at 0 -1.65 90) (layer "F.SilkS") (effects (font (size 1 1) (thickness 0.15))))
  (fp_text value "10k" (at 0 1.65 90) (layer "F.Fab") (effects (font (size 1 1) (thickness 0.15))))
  (pad "1" smd roundrect (at -0.9125 0 270) (size 1.025 1.4) (layers "F.Cu" "F.Paste" "F.Mask") (roundrect_rratio 0.243902) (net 29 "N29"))
  (pad "2" smd roundrect (at 0.9125 0 270) (size 1.025 1.4) (layers "F.Cu" "F.Paste" "F.Mask") (roundrect_rratio 0.243902) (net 1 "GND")))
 (gr_line (start 149.5 66) (end 180 66) (stroke (width 0.1) (type default)) (layer "Edge.Cuts"))
 (gr_arc (start 174.95 64.8) (mid 178.5916 66.3084) (end 180.1 69.95) (stroke (width 0.1) (type default)) (layer "Edge.Cuts"))
 (gr_line (start 180 105) (end 110 105) (stroke (width 0.1) (type default)) (layer "Edge.Cuts"))
 (gr_line (start 156.1 89.55) (end 156.1 88.55) (stroke (width 0.1) (type default)) (layer "Edge.Cuts"))
 (gr_line (start 110 105) (end 110 67) (stroke (width 0.1) (type default)) (layer "Edge.Cuts"))
 (gr_line (start 110.5 66) (end 149.5 66) (stroke (width 0.1) (type default)) (layer "Edge.Cuts"))
 (gr_line (start 156.1 88.55) (end 156.6 88.55) (stroke (width 0.1) (type default)) (layer "Edge.Cuts"))
 (gr_arc (start 180.05 100.05) (mid 178.600179 103.550179) (end 175.1 105) (stroke (width 0.1) (type default)) (layer "Edge.Cuts"))
 (gr_line (start 180 66) (end 180 105) (stroke (width 0.1) (type default)) (layer "Edge.Cuts"))
 (segment (start 175.395 78.8125) (end 173.745 78.8125) (width 0.381) (layer "F.Cu") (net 6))
 (segment (start 172.345 67.2125) (end 172.345 69.6125) (width 0.381) (layer "F.Cu") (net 6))
 (segment (start 176.595 77.6125) (end 175.395 78.8125) (width 0.381) (layer "F.Cu") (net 6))
 (segment (start 176.3625 67.2125) (end 176.75 67.6) (width 0.381) (layer "F.Cu") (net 6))
 (segment (start 165.645 84.205) (end 165.45 84.4) (width 0.381) (layer "F.Cu") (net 6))
 (segment (start 165.645 81.3125) (end 165.645 84.205) (width 0.381) (layer "F.Cu") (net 6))
 (segment (start 167.35 101.8) (end 167.35 100.469) (width 0.381) (layer "F.Cu") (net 6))
 (segment (start 156.05 70.1) (end 158.6375 67.5125) (width 0.381) (layer "F.Cu") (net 6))
 (segment (start 162.345 76.4125) (end 163.476 76.4125) (width 0.381) (layer "F.Cu") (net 6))
 (segment (start 163.795 67.5125) (end 163.795 68.495) (width 0.381) (layer "F.Cu") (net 6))
 (segment (start 167.35 100.469) (end 162.381 95.5) (width 0.381) (layer "F.Cu") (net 6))
 (segment (start 164.15 69.8075) (end 164.045 69.9125) (width 0.381) (layer "F.Cu") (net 6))
 (segment (start 164.15 68.85) (end 164.15 69.8075) (width 0.381) (layer "F.Cu") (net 6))
 (segment (start 163.795 68.495) (end 164.15 68.85) (width 0.381) (layer "F.Cu") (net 6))
 (segment (start 172.345 69.6125) (end 172.045 69.9125) (width 0.381) (layer "F.Cu") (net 6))
 (segment (start 163.476 76.4125) (end 165.645 78.5815) (width 0.381) (layer "F.Cu") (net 6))
 (segment (start 165.645 78.5815) (end 165.645 81.3125) (width 0.381) (layer "F.Cu") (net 6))
 (segment (start 156.05 70.1) (end 158.3625 72.4125) (width 0.381) (layer "F.Cu") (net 6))
 (segment (start 158.6375 67.5125) (end 163.795 67.5125) (width 0.381) (layer "F.Cu") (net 6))
 (segment (start 158.3625 72.4125) (end 162.345 72.4125) (width 0.381) (layer "F.Cu") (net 6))
 (segment (start 162.381 95.5) (end 160.35 95.5) (width 0.381) (layer "F.Cu") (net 6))
 (segment (start 172.345 67.2125) (end 176.3625 67.2125) (width 0.381) (layer "F.Cu") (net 6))
 (via (at 176.75 67.6) (size 0.8) (drill 0.4) (layers "F.Cu" "B.Cu") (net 6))
 (via (at 165.45 84.4) (size 0.8) (drill 0.4) (layers "F.Cu" "B.Cu") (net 6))
 (via (at 162.381 95.5) (size 0.8) (drill 0.4) (layers "F.Cu" "B.Cu") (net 6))
 (segment (start 162.381 87.469) (end 165.45 84.4) (width 0.381) (layer "B.Cu") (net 6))
 (segment (start 162.381 95.5) (end 162.381 87.469) (width 0.381) (layer "B.Cu") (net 6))
 (segment (start 173.75 99.95) (end 178.25 99.95) (width 0.381) (layer "F.Cu") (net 1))
 (segment (start 154.15 70.1) (end 154.15 72.45) (width 0.381) (layer "F.Cu") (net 1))
 (segment (start 165.695 67.5125) (end 170.145 67.5125) (width 0.381) (layer "F.Cu") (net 1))
 (segment (start 164.61925 76.08075) (end 164.845 75.855) (width 0.381) (layer "F.Cu") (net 1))
 (segment (start 164.0155 103.0655) (end 171.1345 103.0655) (width 0.381) (layer "F.Cu") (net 1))
 (segment (start 176.645 73.7625) (end 178.2 75.3175) (width 0.381) (layer "F.Cu") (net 1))
 (segment (start 166.445 85.955) (end 166.445 81.3125) (width 0.381) (layer "F.Cu") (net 1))
 (segment (start 171.3 90.1) (end 170 88.8) (width 0.381) (layer "F.Cu") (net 1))
 (segment (start 167.6 88.7) (end 167.6 90.1) (width 0.381) (layer "F.Cu") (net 1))
 (segment (start 166.445 77.9065) (end 164.61925 76.08075) (width 0.381) (layer "F.Cu") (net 1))
 (segment (start 173.75 92.55) (end 171.3 90.1) (width 0.381) (layer "F.Cu") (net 1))
 (segment (start 170.145 67.5125) (end 170.445 67.2125) (width 0.381) (layer "F.Cu") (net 1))
 (segment (start 162.05 101.1) (end 164.0155 103.0655) (width 0.381) (layer "F.Cu") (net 1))
 (segment (start 166.9075 79.6125) (end 173.745 79.6125) (width 0.381) (layer "F.Cu") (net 1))
 (segment (start 173.745 79.6125) (end 176.495 79.6125) (width 0.381) (layer "F.Cu") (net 1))
 (segment (start 160.05 76.4) (end 160.05 75.5) (width 0.381) (layer "F.Cu") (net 1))
 (segment (start 166.519 88.7) (end 167.6 88.7) (width 0.381) (layer "F.Cu") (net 1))
 (segment (start 154.15 72.45) (end 154.15 75.55) (width 0.381) (layer "F.Cu") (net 1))
 (segment (start 164.845 73.1) (end 164.845 69.9125) (width 0.381) (layer "F.Cu") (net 1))
 (segment (start 164.845 73.1) (end 169.0635 73.1) (width 0.381) (layer "F.Cu") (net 1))
 (segment (start 166.4905 87.0095) (end 166.4905 88.6715) (width 0.381) (layer "F.Cu") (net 1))
 (segment (start 160.05 75.5) (end 160.7375 74.8125) (width 0.381) (layer "F.Cu") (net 1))
 (segment (start 171.245 70.9185) (end 171.245 69.9125) (width 0.381) (layer "F.Cu") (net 1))
 (segment (start 165.4 87) (end 166.481 87) (width 0.381) (layer "F.Cu") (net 1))
 (segment (start 178.2 75.3175) (end 178.2 77.9075) (width 0.381) (layer "F.Cu") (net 1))
 (segment (start 170 88.8) (end 167.7 88.8) (width 0.381) (layer "F.Cu") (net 1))
 (segment (start 169.0635 73.1) (end 171.245 70.9185) (width 0.381) (layer "F.Cu") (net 1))
 (segment (start 173.75 92.65) (end 173.75 92.55) (width 0.381) (layer "F.Cu") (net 1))
 (segment (start 170.445 67.2125) (end 171.245 68.0125) (width 0.381) (layer "F.Cu") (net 1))
 (segment (start 154.15 75.55) (end 155 76.4) (width 0.381) (layer "F.Cu") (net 1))
 (segment (start 173.75 92.65) (end 178.25 92.65) (width 0.381) (layer "F.Cu") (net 1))
 (segment (start 173.75 100.45) (end 173.75 99.95) (width 0.381) (layer "F.Cu") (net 1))
 (segment (start 163.1 88.8) (end 164.4 90.1) (width 0.381) (layer "F.Cu") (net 1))
 (segment (start 166.445 81.3125) (end 166.445 79.15) (width 0.381) (layer "F.Cu") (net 1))
 (segment (start 163.351 74.8125) (end 162.345 74.8125) (width 0.381) (layer "F.Cu") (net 1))
 (segment (start 167.6 90.1) (end 171.3 90.1) (width 0.381) (layer "F.Cu") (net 1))
 (segment (start 165.4 87) (end 166.445 85.955) (width 0.381) (layer "F.Cu") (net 1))
 (segment (start 164.845 75.855) (end 164.845 73.1) (width 0.381) (layer "F.Cu") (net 1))
 (segment (start 171.245 68.0125) (end 171.245 69.9125) (width 0.381) (layer "F.Cu") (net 1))
 (segment (start 166.481 87) (end 166.4905 87.0095) (width 0.381) (layer "F.Cu") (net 1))
 (segment (start 160.7375 74.8125) (end 162.345 74.8125) (width 0.381) (layer "F.Cu") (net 1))
 (segment (start 166.445 79.15) (end 166.445 77.9065) (width 0.381) (layer "F.Cu") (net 1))
 (segment (start 167.7 88.8) (end 167.6 88.7) (width 0.381) (layer "F.Cu") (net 1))
 (segment (start 164.4 90.1) (end 167.6 90.1) (width 0.381) (layer "F.Cu") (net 1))
 (segment (start 178.2 77.9075) (end 176.595 79.5125) (width 0.381) (layer "F.Cu") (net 1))
 (segment (start 166.445 79.15) (end 166.9075 79.6125) (width 0.381) (layer "F.Cu") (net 1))
 (segment (start 176.495 79.6125) (end 176.595 79.5125) (width 0.381) (layer "F.Cu") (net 1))
 (segment (start 166.4905 88.6715) (end 166.519 88.7) (width 0.381) (layer "F.Cu") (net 1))
 (segment (start 171.1345 103.0655) (end 173.75 100.45) (width 0.381) (layer "F.Cu") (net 1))
 (segment (start 164.61925 76.08075) (end 163.351 74.8125) (width 0.381) (layer "F.Cu") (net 1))
 (via (at 160.05 76.4) (size 0.8) (drill 0.4) (layers "F.Cu" "B.Cu") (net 1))
 (via (at 155 76.4) (size 0.8) (drill 0.4) (layers "F.Cu" "B.Cu") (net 1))
 (segment (start 160.05 76.4) (end 155 76.4) (width 0.381) (layer "B.Cu") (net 1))
 (segment (start 169.9 87) (end 170 86.9) (width 0.254) (layer "F.Cu") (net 2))
 (segment (start 167.6 87) (end 168.045 86.555) (width 0.254) (layer "F.Cu") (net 2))
 (segment (start 168.045 86.555) (end 168.045 81.3125) (width 0.254) (layer "F.Cu") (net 2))
 (segment (start 167.6 87) (end 169.9 87) (width 0.254) (layer "F.Cu") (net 2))
 (segment (start 163.1 86.9) (end 163.1 85.25) (width 0.254) (layer "F.Cu") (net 15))
 (segment (start 163.1 85.25) (end 163.4 84.95) (width 0.254) (layer "F.Cu") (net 15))
 (segment (start 163.1 86.9) (end 164.9 88.7) (width 0.254) (layer "F.Cu") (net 15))
 (segment (start 164.9 88.7) (end 165.4 88.7) (width 0.254) (layer "F.Cu") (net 15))
 (segment (start 167.245 83.6265) (end 167.3185 83.7) (width 0.254) (layer "F.Cu") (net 15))
 (segment (start 167.245 81.3125) (end 167.245 83.6265) (width 0.254) (layer "F.Cu") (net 15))
 (via (at 167.3185 83.7) (size 0.8) (drill 0.4) (layers "F.Cu" "B.Cu") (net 15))
 (via (at 163.4 84.95) (size 0.8) (drill 0.4) (layers "F.Cu" "B.Cu") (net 15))
 (segment (start 163.4 84.95) (end 164.677 83.673) (width 0.254) (layer "B.Cu") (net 15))
 (segment (start 164.677 83.673) (end 167.323 83.673) (width 0.254) (layer "B.Cu") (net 15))
 (segment (start 167.35 83.7) (end 167.3185 83.7) (width 0.254) (layer "B.Cu") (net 15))
 (segment (start 167.323 83.673) (end 167.35 83.7) (width 0.254) (layer "B.Cu") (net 15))
 (segment (start 161.6055 75.6125) (end 162.345 75.6125) (width 0.254) (layer "F.Cu") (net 8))
 (segment (start 161.268 77.232) (end 161.268 75.95) (width 0.254) (layer "F.Cu") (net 8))
 (segment (start 160.75 77.75) (end 161.268 77.232) (width 0.254) (layer "F.Cu") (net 8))
 (segment (start 161.268 75.95) (end 161.6055 75.6125) (width 0.254) (layer "F.Cu") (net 8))
 (segment (start 156.05 72.45) (end 156.55 72.95) (width 0.254) (layer "F.Cu") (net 8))
 (segment (start 156.55 72.95) (end 156.55 78.05) (width 0.254) (layer "F.Cu") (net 8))
 (via (at 156.55 78.05) (size 0.8) (drill 0.4) (layers "F.Cu" "B.Cu") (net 8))
 (via (at 160.75 77.75) (size 0.8) (drill 0.4) (layers "F.Cu" "B.Cu") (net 8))
 (segment (start 156.55 78.05) (end 160.45 78.05) (width 0.254) (layer "B.Cu") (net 8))
 (segment (start 160.45 78.05) (end 160.75 77.75) (width 0.254) (layer "B.Cu") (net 8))
 (segment (start 146.2741 97.6334) (end 147.645 96.2625) (width 0.254) (layer "F.Cu") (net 40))
 (segment (start 128.245 95.8125) (end 130.0659 97.6334) (width 0.254) (layer "F.Cu") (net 40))
 (segment (start 130.0659 97.6334) (end 146.2741 97.6334) (width 0.254) (layer "F.Cu") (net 40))
 (segment (start 125.915 90.1825) (end 128.245 92.5125) (width 0.254) (layer "F.Cu") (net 47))
 (segment (start 122.885 90.1825) (end 125.915 90.1825) (width 0.254) (layer "F.Cu") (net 47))
 (segment (start 142.095 90.7625) (end 145.445 90.7625) (width 0.254) (layer "F.Cu") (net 41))
 (segment (start 145.445 90.7625) (end 147.645 92.9625) (width 0.254) (layer "F.Cu") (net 41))
 (segment (start 145.9741 78.4334) (end 147.795 76.6125) (width 0.254) (layer "F.Cu") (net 37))
 (segment (start 130.3659 78.4334) (end 145.9741 78.4334) (width 0.254) (layer "F.Cu") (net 37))
 (segment (start 128.495 76.5625) (end 130.3659 78.4334) (width 0.254) (layer "F.Cu") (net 37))
 (segment (start 126.7825 71.55) (end 128.495 73.2625) (width 0.254) (layer "F.Cu") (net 38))
 (segment (start 122.9 71.55) (end 126.7825 71.55) (width 0.254) (layer "F.Cu") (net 38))
 (segment (start 142.195 71.5625) (end 146.045 71.5625) (width 0.254) (layer "F.Cu") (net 44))
 (segment (start 146.045 71.5625) (end 147.795 73.3125) (width 0.254) (layer "F.Cu") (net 44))
 (segment (start 172.875 97.9) (end 173.75 97.9) (width 0.254) (layer "F.Cu") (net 45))
 (segment (start 170.15 100.625) (end 172.875 97.9) (width 0.254) (layer "F.Cu") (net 45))
 (segment (start 170.15 101.8) (end 170.15 100.625) (width 0.254) (layer "F.Cu") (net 45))
 (segment (start 116.59 73.51) (end 116.59 92.6675) (width 0.254) (layer "F.Cu") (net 39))
 (segment (start 116.59 92.6675) (end 116.535 92.7225) (width 0.254) (layer "F.Cu") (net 39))
 (segment (start 137.095 74.7325) (end 137.095 91.2625) (width 0.254) (layer "B.Cu") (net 43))
 (segment (start 135.885 73.5225) (end 137.095 74.7325) (width 0.254) (layer "B.Cu") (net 43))
 (segment (start 176.645 71.9375) (end 176.32 71.6125) (width 0.254) (layer "F.Cu") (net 29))
 (segment (start 176.32 71.6125) (end 173.745 71.6125) (width 0.254) (layer "F.Cu") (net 29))
 (segment (start 159.3 89.55) (end 159.3 78.45) (width 0.254) (layer "F.Cu") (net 7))
 (segment (start 165.25 95.5) (end 159.3 89.55) (width 0.254) (layer "F.Cu") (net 7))
 (segment (start 160.5875 74.0125) (end 162.345 74.0125) (width 0.254) (layer "F.Cu") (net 7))
 (segment (start 159.3 78.45) (end 159.3 75.3) (width 0.254) (layer "F.Cu") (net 7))
 (segment (start 168.8875 95.5) (end 165.25 95.5) (width 0.254) (layer "F.Cu") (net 7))
 (segment (start 159.3 75.3) (end 160.5875 74.0125) (width 0.254) (layer "F.Cu") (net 7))
 (segment (start 173.75 96.3) (end 172.425 96.3) (width 0.2) (layer "F.Cu") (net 42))
 (segment (start 172.425 96.3) (end 171.625 95.5) (width 0.2) (layer "F.Cu") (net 42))
 (segment (start 171.625 95.5) (end 170.7125 95.5) (width 0.2) (layer "F.Cu") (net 42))
 (segment (start 172.425 97.1) (end 171.575 97.95) (width 0.2) (layer "F.Cu") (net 3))
 (segment (start 173.75 97.1) (end 172.425 97.1) (width 0.2) (layer "F.Cu") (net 3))
 (segment (start 171.575 97.95) (end 170.7125 97.95) (width 0.2) (layer "F.Cu") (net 3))
 (segment (start 158 89.6) (end 158 75.55) (width 0.254) (layer "F.Cu") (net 4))
 (segment (start 166.35 97.95) (end 159.325 90.925) (width 0.254) (layer "F.Cu") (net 4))
 (segment (start 159.325 90.925) (end 158 89.6) (width 0.254) (layer "F.Cu") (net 4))
 (segment (start 159.325 90.925) (end 159.2 90.8) (width 0.254) (layer "F.Cu") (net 4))
 (segment (start 168.8875 97.95) (end 166.35 97.95) (width 0.254) (layer "F.Cu") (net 4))
 (segment (start 160.3375 73.2125) (end 162.345 73.2125) (width 0.254) (layer "F.Cu") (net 4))
 (segment (start 158 75.55) (end 160.3375 73.2125) (width 0.254) (layer "F.Cu") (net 4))
 (segment (start 158.525 95.5) (end 158.525 93.525) (width 0.254) (layer "F.Cu") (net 14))
 (segment (start 162.6115 84.55) (end 164.845 82.3165) (width 0.254) (layer "F.Cu") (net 14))
 (segment (start 164.845 82.3165) (end 164.845 81.3125) (width 0.254) (layer "F.Cu") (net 14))
 (segment (start 161.3 84.55) (end 162.6115 84.55) (width 0.254) (layer "F.Cu") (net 14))
 (segment (start 157.75 95.5) (end 158.525 95.5) (width 0.254) (layer "F.Cu") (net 14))
 (segment (start 155.85 97.4) (end 157.75 95.5) (width 0.254) (layer "F.Cu") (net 14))
 (segment (start 158.525 93.525) (end 159.15 92.9) (width 0.254) (layer "F.Cu") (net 14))
 (segment (start 159.15 92.9) (end 159.35 92.7) (width 0.254) (layer "F.Cu") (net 14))
 (via (at 161.3 84.55) (size 0.8) (drill 0.4) (layers "F.Cu" "B.Cu") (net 14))
 (via (at 159.35 92.7) (size 0.8) (drill 0.4) (layers "F.Cu" "B.Cu") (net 14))
 (segment (start 161.3 90.75) (end 161.3 84.55) (width 0.254) (layer "B.Cu") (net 14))
 (segment (start 159.35 92.7) (end 161.3 90.75) (width 0.254) (layer "B.Cu") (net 14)))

